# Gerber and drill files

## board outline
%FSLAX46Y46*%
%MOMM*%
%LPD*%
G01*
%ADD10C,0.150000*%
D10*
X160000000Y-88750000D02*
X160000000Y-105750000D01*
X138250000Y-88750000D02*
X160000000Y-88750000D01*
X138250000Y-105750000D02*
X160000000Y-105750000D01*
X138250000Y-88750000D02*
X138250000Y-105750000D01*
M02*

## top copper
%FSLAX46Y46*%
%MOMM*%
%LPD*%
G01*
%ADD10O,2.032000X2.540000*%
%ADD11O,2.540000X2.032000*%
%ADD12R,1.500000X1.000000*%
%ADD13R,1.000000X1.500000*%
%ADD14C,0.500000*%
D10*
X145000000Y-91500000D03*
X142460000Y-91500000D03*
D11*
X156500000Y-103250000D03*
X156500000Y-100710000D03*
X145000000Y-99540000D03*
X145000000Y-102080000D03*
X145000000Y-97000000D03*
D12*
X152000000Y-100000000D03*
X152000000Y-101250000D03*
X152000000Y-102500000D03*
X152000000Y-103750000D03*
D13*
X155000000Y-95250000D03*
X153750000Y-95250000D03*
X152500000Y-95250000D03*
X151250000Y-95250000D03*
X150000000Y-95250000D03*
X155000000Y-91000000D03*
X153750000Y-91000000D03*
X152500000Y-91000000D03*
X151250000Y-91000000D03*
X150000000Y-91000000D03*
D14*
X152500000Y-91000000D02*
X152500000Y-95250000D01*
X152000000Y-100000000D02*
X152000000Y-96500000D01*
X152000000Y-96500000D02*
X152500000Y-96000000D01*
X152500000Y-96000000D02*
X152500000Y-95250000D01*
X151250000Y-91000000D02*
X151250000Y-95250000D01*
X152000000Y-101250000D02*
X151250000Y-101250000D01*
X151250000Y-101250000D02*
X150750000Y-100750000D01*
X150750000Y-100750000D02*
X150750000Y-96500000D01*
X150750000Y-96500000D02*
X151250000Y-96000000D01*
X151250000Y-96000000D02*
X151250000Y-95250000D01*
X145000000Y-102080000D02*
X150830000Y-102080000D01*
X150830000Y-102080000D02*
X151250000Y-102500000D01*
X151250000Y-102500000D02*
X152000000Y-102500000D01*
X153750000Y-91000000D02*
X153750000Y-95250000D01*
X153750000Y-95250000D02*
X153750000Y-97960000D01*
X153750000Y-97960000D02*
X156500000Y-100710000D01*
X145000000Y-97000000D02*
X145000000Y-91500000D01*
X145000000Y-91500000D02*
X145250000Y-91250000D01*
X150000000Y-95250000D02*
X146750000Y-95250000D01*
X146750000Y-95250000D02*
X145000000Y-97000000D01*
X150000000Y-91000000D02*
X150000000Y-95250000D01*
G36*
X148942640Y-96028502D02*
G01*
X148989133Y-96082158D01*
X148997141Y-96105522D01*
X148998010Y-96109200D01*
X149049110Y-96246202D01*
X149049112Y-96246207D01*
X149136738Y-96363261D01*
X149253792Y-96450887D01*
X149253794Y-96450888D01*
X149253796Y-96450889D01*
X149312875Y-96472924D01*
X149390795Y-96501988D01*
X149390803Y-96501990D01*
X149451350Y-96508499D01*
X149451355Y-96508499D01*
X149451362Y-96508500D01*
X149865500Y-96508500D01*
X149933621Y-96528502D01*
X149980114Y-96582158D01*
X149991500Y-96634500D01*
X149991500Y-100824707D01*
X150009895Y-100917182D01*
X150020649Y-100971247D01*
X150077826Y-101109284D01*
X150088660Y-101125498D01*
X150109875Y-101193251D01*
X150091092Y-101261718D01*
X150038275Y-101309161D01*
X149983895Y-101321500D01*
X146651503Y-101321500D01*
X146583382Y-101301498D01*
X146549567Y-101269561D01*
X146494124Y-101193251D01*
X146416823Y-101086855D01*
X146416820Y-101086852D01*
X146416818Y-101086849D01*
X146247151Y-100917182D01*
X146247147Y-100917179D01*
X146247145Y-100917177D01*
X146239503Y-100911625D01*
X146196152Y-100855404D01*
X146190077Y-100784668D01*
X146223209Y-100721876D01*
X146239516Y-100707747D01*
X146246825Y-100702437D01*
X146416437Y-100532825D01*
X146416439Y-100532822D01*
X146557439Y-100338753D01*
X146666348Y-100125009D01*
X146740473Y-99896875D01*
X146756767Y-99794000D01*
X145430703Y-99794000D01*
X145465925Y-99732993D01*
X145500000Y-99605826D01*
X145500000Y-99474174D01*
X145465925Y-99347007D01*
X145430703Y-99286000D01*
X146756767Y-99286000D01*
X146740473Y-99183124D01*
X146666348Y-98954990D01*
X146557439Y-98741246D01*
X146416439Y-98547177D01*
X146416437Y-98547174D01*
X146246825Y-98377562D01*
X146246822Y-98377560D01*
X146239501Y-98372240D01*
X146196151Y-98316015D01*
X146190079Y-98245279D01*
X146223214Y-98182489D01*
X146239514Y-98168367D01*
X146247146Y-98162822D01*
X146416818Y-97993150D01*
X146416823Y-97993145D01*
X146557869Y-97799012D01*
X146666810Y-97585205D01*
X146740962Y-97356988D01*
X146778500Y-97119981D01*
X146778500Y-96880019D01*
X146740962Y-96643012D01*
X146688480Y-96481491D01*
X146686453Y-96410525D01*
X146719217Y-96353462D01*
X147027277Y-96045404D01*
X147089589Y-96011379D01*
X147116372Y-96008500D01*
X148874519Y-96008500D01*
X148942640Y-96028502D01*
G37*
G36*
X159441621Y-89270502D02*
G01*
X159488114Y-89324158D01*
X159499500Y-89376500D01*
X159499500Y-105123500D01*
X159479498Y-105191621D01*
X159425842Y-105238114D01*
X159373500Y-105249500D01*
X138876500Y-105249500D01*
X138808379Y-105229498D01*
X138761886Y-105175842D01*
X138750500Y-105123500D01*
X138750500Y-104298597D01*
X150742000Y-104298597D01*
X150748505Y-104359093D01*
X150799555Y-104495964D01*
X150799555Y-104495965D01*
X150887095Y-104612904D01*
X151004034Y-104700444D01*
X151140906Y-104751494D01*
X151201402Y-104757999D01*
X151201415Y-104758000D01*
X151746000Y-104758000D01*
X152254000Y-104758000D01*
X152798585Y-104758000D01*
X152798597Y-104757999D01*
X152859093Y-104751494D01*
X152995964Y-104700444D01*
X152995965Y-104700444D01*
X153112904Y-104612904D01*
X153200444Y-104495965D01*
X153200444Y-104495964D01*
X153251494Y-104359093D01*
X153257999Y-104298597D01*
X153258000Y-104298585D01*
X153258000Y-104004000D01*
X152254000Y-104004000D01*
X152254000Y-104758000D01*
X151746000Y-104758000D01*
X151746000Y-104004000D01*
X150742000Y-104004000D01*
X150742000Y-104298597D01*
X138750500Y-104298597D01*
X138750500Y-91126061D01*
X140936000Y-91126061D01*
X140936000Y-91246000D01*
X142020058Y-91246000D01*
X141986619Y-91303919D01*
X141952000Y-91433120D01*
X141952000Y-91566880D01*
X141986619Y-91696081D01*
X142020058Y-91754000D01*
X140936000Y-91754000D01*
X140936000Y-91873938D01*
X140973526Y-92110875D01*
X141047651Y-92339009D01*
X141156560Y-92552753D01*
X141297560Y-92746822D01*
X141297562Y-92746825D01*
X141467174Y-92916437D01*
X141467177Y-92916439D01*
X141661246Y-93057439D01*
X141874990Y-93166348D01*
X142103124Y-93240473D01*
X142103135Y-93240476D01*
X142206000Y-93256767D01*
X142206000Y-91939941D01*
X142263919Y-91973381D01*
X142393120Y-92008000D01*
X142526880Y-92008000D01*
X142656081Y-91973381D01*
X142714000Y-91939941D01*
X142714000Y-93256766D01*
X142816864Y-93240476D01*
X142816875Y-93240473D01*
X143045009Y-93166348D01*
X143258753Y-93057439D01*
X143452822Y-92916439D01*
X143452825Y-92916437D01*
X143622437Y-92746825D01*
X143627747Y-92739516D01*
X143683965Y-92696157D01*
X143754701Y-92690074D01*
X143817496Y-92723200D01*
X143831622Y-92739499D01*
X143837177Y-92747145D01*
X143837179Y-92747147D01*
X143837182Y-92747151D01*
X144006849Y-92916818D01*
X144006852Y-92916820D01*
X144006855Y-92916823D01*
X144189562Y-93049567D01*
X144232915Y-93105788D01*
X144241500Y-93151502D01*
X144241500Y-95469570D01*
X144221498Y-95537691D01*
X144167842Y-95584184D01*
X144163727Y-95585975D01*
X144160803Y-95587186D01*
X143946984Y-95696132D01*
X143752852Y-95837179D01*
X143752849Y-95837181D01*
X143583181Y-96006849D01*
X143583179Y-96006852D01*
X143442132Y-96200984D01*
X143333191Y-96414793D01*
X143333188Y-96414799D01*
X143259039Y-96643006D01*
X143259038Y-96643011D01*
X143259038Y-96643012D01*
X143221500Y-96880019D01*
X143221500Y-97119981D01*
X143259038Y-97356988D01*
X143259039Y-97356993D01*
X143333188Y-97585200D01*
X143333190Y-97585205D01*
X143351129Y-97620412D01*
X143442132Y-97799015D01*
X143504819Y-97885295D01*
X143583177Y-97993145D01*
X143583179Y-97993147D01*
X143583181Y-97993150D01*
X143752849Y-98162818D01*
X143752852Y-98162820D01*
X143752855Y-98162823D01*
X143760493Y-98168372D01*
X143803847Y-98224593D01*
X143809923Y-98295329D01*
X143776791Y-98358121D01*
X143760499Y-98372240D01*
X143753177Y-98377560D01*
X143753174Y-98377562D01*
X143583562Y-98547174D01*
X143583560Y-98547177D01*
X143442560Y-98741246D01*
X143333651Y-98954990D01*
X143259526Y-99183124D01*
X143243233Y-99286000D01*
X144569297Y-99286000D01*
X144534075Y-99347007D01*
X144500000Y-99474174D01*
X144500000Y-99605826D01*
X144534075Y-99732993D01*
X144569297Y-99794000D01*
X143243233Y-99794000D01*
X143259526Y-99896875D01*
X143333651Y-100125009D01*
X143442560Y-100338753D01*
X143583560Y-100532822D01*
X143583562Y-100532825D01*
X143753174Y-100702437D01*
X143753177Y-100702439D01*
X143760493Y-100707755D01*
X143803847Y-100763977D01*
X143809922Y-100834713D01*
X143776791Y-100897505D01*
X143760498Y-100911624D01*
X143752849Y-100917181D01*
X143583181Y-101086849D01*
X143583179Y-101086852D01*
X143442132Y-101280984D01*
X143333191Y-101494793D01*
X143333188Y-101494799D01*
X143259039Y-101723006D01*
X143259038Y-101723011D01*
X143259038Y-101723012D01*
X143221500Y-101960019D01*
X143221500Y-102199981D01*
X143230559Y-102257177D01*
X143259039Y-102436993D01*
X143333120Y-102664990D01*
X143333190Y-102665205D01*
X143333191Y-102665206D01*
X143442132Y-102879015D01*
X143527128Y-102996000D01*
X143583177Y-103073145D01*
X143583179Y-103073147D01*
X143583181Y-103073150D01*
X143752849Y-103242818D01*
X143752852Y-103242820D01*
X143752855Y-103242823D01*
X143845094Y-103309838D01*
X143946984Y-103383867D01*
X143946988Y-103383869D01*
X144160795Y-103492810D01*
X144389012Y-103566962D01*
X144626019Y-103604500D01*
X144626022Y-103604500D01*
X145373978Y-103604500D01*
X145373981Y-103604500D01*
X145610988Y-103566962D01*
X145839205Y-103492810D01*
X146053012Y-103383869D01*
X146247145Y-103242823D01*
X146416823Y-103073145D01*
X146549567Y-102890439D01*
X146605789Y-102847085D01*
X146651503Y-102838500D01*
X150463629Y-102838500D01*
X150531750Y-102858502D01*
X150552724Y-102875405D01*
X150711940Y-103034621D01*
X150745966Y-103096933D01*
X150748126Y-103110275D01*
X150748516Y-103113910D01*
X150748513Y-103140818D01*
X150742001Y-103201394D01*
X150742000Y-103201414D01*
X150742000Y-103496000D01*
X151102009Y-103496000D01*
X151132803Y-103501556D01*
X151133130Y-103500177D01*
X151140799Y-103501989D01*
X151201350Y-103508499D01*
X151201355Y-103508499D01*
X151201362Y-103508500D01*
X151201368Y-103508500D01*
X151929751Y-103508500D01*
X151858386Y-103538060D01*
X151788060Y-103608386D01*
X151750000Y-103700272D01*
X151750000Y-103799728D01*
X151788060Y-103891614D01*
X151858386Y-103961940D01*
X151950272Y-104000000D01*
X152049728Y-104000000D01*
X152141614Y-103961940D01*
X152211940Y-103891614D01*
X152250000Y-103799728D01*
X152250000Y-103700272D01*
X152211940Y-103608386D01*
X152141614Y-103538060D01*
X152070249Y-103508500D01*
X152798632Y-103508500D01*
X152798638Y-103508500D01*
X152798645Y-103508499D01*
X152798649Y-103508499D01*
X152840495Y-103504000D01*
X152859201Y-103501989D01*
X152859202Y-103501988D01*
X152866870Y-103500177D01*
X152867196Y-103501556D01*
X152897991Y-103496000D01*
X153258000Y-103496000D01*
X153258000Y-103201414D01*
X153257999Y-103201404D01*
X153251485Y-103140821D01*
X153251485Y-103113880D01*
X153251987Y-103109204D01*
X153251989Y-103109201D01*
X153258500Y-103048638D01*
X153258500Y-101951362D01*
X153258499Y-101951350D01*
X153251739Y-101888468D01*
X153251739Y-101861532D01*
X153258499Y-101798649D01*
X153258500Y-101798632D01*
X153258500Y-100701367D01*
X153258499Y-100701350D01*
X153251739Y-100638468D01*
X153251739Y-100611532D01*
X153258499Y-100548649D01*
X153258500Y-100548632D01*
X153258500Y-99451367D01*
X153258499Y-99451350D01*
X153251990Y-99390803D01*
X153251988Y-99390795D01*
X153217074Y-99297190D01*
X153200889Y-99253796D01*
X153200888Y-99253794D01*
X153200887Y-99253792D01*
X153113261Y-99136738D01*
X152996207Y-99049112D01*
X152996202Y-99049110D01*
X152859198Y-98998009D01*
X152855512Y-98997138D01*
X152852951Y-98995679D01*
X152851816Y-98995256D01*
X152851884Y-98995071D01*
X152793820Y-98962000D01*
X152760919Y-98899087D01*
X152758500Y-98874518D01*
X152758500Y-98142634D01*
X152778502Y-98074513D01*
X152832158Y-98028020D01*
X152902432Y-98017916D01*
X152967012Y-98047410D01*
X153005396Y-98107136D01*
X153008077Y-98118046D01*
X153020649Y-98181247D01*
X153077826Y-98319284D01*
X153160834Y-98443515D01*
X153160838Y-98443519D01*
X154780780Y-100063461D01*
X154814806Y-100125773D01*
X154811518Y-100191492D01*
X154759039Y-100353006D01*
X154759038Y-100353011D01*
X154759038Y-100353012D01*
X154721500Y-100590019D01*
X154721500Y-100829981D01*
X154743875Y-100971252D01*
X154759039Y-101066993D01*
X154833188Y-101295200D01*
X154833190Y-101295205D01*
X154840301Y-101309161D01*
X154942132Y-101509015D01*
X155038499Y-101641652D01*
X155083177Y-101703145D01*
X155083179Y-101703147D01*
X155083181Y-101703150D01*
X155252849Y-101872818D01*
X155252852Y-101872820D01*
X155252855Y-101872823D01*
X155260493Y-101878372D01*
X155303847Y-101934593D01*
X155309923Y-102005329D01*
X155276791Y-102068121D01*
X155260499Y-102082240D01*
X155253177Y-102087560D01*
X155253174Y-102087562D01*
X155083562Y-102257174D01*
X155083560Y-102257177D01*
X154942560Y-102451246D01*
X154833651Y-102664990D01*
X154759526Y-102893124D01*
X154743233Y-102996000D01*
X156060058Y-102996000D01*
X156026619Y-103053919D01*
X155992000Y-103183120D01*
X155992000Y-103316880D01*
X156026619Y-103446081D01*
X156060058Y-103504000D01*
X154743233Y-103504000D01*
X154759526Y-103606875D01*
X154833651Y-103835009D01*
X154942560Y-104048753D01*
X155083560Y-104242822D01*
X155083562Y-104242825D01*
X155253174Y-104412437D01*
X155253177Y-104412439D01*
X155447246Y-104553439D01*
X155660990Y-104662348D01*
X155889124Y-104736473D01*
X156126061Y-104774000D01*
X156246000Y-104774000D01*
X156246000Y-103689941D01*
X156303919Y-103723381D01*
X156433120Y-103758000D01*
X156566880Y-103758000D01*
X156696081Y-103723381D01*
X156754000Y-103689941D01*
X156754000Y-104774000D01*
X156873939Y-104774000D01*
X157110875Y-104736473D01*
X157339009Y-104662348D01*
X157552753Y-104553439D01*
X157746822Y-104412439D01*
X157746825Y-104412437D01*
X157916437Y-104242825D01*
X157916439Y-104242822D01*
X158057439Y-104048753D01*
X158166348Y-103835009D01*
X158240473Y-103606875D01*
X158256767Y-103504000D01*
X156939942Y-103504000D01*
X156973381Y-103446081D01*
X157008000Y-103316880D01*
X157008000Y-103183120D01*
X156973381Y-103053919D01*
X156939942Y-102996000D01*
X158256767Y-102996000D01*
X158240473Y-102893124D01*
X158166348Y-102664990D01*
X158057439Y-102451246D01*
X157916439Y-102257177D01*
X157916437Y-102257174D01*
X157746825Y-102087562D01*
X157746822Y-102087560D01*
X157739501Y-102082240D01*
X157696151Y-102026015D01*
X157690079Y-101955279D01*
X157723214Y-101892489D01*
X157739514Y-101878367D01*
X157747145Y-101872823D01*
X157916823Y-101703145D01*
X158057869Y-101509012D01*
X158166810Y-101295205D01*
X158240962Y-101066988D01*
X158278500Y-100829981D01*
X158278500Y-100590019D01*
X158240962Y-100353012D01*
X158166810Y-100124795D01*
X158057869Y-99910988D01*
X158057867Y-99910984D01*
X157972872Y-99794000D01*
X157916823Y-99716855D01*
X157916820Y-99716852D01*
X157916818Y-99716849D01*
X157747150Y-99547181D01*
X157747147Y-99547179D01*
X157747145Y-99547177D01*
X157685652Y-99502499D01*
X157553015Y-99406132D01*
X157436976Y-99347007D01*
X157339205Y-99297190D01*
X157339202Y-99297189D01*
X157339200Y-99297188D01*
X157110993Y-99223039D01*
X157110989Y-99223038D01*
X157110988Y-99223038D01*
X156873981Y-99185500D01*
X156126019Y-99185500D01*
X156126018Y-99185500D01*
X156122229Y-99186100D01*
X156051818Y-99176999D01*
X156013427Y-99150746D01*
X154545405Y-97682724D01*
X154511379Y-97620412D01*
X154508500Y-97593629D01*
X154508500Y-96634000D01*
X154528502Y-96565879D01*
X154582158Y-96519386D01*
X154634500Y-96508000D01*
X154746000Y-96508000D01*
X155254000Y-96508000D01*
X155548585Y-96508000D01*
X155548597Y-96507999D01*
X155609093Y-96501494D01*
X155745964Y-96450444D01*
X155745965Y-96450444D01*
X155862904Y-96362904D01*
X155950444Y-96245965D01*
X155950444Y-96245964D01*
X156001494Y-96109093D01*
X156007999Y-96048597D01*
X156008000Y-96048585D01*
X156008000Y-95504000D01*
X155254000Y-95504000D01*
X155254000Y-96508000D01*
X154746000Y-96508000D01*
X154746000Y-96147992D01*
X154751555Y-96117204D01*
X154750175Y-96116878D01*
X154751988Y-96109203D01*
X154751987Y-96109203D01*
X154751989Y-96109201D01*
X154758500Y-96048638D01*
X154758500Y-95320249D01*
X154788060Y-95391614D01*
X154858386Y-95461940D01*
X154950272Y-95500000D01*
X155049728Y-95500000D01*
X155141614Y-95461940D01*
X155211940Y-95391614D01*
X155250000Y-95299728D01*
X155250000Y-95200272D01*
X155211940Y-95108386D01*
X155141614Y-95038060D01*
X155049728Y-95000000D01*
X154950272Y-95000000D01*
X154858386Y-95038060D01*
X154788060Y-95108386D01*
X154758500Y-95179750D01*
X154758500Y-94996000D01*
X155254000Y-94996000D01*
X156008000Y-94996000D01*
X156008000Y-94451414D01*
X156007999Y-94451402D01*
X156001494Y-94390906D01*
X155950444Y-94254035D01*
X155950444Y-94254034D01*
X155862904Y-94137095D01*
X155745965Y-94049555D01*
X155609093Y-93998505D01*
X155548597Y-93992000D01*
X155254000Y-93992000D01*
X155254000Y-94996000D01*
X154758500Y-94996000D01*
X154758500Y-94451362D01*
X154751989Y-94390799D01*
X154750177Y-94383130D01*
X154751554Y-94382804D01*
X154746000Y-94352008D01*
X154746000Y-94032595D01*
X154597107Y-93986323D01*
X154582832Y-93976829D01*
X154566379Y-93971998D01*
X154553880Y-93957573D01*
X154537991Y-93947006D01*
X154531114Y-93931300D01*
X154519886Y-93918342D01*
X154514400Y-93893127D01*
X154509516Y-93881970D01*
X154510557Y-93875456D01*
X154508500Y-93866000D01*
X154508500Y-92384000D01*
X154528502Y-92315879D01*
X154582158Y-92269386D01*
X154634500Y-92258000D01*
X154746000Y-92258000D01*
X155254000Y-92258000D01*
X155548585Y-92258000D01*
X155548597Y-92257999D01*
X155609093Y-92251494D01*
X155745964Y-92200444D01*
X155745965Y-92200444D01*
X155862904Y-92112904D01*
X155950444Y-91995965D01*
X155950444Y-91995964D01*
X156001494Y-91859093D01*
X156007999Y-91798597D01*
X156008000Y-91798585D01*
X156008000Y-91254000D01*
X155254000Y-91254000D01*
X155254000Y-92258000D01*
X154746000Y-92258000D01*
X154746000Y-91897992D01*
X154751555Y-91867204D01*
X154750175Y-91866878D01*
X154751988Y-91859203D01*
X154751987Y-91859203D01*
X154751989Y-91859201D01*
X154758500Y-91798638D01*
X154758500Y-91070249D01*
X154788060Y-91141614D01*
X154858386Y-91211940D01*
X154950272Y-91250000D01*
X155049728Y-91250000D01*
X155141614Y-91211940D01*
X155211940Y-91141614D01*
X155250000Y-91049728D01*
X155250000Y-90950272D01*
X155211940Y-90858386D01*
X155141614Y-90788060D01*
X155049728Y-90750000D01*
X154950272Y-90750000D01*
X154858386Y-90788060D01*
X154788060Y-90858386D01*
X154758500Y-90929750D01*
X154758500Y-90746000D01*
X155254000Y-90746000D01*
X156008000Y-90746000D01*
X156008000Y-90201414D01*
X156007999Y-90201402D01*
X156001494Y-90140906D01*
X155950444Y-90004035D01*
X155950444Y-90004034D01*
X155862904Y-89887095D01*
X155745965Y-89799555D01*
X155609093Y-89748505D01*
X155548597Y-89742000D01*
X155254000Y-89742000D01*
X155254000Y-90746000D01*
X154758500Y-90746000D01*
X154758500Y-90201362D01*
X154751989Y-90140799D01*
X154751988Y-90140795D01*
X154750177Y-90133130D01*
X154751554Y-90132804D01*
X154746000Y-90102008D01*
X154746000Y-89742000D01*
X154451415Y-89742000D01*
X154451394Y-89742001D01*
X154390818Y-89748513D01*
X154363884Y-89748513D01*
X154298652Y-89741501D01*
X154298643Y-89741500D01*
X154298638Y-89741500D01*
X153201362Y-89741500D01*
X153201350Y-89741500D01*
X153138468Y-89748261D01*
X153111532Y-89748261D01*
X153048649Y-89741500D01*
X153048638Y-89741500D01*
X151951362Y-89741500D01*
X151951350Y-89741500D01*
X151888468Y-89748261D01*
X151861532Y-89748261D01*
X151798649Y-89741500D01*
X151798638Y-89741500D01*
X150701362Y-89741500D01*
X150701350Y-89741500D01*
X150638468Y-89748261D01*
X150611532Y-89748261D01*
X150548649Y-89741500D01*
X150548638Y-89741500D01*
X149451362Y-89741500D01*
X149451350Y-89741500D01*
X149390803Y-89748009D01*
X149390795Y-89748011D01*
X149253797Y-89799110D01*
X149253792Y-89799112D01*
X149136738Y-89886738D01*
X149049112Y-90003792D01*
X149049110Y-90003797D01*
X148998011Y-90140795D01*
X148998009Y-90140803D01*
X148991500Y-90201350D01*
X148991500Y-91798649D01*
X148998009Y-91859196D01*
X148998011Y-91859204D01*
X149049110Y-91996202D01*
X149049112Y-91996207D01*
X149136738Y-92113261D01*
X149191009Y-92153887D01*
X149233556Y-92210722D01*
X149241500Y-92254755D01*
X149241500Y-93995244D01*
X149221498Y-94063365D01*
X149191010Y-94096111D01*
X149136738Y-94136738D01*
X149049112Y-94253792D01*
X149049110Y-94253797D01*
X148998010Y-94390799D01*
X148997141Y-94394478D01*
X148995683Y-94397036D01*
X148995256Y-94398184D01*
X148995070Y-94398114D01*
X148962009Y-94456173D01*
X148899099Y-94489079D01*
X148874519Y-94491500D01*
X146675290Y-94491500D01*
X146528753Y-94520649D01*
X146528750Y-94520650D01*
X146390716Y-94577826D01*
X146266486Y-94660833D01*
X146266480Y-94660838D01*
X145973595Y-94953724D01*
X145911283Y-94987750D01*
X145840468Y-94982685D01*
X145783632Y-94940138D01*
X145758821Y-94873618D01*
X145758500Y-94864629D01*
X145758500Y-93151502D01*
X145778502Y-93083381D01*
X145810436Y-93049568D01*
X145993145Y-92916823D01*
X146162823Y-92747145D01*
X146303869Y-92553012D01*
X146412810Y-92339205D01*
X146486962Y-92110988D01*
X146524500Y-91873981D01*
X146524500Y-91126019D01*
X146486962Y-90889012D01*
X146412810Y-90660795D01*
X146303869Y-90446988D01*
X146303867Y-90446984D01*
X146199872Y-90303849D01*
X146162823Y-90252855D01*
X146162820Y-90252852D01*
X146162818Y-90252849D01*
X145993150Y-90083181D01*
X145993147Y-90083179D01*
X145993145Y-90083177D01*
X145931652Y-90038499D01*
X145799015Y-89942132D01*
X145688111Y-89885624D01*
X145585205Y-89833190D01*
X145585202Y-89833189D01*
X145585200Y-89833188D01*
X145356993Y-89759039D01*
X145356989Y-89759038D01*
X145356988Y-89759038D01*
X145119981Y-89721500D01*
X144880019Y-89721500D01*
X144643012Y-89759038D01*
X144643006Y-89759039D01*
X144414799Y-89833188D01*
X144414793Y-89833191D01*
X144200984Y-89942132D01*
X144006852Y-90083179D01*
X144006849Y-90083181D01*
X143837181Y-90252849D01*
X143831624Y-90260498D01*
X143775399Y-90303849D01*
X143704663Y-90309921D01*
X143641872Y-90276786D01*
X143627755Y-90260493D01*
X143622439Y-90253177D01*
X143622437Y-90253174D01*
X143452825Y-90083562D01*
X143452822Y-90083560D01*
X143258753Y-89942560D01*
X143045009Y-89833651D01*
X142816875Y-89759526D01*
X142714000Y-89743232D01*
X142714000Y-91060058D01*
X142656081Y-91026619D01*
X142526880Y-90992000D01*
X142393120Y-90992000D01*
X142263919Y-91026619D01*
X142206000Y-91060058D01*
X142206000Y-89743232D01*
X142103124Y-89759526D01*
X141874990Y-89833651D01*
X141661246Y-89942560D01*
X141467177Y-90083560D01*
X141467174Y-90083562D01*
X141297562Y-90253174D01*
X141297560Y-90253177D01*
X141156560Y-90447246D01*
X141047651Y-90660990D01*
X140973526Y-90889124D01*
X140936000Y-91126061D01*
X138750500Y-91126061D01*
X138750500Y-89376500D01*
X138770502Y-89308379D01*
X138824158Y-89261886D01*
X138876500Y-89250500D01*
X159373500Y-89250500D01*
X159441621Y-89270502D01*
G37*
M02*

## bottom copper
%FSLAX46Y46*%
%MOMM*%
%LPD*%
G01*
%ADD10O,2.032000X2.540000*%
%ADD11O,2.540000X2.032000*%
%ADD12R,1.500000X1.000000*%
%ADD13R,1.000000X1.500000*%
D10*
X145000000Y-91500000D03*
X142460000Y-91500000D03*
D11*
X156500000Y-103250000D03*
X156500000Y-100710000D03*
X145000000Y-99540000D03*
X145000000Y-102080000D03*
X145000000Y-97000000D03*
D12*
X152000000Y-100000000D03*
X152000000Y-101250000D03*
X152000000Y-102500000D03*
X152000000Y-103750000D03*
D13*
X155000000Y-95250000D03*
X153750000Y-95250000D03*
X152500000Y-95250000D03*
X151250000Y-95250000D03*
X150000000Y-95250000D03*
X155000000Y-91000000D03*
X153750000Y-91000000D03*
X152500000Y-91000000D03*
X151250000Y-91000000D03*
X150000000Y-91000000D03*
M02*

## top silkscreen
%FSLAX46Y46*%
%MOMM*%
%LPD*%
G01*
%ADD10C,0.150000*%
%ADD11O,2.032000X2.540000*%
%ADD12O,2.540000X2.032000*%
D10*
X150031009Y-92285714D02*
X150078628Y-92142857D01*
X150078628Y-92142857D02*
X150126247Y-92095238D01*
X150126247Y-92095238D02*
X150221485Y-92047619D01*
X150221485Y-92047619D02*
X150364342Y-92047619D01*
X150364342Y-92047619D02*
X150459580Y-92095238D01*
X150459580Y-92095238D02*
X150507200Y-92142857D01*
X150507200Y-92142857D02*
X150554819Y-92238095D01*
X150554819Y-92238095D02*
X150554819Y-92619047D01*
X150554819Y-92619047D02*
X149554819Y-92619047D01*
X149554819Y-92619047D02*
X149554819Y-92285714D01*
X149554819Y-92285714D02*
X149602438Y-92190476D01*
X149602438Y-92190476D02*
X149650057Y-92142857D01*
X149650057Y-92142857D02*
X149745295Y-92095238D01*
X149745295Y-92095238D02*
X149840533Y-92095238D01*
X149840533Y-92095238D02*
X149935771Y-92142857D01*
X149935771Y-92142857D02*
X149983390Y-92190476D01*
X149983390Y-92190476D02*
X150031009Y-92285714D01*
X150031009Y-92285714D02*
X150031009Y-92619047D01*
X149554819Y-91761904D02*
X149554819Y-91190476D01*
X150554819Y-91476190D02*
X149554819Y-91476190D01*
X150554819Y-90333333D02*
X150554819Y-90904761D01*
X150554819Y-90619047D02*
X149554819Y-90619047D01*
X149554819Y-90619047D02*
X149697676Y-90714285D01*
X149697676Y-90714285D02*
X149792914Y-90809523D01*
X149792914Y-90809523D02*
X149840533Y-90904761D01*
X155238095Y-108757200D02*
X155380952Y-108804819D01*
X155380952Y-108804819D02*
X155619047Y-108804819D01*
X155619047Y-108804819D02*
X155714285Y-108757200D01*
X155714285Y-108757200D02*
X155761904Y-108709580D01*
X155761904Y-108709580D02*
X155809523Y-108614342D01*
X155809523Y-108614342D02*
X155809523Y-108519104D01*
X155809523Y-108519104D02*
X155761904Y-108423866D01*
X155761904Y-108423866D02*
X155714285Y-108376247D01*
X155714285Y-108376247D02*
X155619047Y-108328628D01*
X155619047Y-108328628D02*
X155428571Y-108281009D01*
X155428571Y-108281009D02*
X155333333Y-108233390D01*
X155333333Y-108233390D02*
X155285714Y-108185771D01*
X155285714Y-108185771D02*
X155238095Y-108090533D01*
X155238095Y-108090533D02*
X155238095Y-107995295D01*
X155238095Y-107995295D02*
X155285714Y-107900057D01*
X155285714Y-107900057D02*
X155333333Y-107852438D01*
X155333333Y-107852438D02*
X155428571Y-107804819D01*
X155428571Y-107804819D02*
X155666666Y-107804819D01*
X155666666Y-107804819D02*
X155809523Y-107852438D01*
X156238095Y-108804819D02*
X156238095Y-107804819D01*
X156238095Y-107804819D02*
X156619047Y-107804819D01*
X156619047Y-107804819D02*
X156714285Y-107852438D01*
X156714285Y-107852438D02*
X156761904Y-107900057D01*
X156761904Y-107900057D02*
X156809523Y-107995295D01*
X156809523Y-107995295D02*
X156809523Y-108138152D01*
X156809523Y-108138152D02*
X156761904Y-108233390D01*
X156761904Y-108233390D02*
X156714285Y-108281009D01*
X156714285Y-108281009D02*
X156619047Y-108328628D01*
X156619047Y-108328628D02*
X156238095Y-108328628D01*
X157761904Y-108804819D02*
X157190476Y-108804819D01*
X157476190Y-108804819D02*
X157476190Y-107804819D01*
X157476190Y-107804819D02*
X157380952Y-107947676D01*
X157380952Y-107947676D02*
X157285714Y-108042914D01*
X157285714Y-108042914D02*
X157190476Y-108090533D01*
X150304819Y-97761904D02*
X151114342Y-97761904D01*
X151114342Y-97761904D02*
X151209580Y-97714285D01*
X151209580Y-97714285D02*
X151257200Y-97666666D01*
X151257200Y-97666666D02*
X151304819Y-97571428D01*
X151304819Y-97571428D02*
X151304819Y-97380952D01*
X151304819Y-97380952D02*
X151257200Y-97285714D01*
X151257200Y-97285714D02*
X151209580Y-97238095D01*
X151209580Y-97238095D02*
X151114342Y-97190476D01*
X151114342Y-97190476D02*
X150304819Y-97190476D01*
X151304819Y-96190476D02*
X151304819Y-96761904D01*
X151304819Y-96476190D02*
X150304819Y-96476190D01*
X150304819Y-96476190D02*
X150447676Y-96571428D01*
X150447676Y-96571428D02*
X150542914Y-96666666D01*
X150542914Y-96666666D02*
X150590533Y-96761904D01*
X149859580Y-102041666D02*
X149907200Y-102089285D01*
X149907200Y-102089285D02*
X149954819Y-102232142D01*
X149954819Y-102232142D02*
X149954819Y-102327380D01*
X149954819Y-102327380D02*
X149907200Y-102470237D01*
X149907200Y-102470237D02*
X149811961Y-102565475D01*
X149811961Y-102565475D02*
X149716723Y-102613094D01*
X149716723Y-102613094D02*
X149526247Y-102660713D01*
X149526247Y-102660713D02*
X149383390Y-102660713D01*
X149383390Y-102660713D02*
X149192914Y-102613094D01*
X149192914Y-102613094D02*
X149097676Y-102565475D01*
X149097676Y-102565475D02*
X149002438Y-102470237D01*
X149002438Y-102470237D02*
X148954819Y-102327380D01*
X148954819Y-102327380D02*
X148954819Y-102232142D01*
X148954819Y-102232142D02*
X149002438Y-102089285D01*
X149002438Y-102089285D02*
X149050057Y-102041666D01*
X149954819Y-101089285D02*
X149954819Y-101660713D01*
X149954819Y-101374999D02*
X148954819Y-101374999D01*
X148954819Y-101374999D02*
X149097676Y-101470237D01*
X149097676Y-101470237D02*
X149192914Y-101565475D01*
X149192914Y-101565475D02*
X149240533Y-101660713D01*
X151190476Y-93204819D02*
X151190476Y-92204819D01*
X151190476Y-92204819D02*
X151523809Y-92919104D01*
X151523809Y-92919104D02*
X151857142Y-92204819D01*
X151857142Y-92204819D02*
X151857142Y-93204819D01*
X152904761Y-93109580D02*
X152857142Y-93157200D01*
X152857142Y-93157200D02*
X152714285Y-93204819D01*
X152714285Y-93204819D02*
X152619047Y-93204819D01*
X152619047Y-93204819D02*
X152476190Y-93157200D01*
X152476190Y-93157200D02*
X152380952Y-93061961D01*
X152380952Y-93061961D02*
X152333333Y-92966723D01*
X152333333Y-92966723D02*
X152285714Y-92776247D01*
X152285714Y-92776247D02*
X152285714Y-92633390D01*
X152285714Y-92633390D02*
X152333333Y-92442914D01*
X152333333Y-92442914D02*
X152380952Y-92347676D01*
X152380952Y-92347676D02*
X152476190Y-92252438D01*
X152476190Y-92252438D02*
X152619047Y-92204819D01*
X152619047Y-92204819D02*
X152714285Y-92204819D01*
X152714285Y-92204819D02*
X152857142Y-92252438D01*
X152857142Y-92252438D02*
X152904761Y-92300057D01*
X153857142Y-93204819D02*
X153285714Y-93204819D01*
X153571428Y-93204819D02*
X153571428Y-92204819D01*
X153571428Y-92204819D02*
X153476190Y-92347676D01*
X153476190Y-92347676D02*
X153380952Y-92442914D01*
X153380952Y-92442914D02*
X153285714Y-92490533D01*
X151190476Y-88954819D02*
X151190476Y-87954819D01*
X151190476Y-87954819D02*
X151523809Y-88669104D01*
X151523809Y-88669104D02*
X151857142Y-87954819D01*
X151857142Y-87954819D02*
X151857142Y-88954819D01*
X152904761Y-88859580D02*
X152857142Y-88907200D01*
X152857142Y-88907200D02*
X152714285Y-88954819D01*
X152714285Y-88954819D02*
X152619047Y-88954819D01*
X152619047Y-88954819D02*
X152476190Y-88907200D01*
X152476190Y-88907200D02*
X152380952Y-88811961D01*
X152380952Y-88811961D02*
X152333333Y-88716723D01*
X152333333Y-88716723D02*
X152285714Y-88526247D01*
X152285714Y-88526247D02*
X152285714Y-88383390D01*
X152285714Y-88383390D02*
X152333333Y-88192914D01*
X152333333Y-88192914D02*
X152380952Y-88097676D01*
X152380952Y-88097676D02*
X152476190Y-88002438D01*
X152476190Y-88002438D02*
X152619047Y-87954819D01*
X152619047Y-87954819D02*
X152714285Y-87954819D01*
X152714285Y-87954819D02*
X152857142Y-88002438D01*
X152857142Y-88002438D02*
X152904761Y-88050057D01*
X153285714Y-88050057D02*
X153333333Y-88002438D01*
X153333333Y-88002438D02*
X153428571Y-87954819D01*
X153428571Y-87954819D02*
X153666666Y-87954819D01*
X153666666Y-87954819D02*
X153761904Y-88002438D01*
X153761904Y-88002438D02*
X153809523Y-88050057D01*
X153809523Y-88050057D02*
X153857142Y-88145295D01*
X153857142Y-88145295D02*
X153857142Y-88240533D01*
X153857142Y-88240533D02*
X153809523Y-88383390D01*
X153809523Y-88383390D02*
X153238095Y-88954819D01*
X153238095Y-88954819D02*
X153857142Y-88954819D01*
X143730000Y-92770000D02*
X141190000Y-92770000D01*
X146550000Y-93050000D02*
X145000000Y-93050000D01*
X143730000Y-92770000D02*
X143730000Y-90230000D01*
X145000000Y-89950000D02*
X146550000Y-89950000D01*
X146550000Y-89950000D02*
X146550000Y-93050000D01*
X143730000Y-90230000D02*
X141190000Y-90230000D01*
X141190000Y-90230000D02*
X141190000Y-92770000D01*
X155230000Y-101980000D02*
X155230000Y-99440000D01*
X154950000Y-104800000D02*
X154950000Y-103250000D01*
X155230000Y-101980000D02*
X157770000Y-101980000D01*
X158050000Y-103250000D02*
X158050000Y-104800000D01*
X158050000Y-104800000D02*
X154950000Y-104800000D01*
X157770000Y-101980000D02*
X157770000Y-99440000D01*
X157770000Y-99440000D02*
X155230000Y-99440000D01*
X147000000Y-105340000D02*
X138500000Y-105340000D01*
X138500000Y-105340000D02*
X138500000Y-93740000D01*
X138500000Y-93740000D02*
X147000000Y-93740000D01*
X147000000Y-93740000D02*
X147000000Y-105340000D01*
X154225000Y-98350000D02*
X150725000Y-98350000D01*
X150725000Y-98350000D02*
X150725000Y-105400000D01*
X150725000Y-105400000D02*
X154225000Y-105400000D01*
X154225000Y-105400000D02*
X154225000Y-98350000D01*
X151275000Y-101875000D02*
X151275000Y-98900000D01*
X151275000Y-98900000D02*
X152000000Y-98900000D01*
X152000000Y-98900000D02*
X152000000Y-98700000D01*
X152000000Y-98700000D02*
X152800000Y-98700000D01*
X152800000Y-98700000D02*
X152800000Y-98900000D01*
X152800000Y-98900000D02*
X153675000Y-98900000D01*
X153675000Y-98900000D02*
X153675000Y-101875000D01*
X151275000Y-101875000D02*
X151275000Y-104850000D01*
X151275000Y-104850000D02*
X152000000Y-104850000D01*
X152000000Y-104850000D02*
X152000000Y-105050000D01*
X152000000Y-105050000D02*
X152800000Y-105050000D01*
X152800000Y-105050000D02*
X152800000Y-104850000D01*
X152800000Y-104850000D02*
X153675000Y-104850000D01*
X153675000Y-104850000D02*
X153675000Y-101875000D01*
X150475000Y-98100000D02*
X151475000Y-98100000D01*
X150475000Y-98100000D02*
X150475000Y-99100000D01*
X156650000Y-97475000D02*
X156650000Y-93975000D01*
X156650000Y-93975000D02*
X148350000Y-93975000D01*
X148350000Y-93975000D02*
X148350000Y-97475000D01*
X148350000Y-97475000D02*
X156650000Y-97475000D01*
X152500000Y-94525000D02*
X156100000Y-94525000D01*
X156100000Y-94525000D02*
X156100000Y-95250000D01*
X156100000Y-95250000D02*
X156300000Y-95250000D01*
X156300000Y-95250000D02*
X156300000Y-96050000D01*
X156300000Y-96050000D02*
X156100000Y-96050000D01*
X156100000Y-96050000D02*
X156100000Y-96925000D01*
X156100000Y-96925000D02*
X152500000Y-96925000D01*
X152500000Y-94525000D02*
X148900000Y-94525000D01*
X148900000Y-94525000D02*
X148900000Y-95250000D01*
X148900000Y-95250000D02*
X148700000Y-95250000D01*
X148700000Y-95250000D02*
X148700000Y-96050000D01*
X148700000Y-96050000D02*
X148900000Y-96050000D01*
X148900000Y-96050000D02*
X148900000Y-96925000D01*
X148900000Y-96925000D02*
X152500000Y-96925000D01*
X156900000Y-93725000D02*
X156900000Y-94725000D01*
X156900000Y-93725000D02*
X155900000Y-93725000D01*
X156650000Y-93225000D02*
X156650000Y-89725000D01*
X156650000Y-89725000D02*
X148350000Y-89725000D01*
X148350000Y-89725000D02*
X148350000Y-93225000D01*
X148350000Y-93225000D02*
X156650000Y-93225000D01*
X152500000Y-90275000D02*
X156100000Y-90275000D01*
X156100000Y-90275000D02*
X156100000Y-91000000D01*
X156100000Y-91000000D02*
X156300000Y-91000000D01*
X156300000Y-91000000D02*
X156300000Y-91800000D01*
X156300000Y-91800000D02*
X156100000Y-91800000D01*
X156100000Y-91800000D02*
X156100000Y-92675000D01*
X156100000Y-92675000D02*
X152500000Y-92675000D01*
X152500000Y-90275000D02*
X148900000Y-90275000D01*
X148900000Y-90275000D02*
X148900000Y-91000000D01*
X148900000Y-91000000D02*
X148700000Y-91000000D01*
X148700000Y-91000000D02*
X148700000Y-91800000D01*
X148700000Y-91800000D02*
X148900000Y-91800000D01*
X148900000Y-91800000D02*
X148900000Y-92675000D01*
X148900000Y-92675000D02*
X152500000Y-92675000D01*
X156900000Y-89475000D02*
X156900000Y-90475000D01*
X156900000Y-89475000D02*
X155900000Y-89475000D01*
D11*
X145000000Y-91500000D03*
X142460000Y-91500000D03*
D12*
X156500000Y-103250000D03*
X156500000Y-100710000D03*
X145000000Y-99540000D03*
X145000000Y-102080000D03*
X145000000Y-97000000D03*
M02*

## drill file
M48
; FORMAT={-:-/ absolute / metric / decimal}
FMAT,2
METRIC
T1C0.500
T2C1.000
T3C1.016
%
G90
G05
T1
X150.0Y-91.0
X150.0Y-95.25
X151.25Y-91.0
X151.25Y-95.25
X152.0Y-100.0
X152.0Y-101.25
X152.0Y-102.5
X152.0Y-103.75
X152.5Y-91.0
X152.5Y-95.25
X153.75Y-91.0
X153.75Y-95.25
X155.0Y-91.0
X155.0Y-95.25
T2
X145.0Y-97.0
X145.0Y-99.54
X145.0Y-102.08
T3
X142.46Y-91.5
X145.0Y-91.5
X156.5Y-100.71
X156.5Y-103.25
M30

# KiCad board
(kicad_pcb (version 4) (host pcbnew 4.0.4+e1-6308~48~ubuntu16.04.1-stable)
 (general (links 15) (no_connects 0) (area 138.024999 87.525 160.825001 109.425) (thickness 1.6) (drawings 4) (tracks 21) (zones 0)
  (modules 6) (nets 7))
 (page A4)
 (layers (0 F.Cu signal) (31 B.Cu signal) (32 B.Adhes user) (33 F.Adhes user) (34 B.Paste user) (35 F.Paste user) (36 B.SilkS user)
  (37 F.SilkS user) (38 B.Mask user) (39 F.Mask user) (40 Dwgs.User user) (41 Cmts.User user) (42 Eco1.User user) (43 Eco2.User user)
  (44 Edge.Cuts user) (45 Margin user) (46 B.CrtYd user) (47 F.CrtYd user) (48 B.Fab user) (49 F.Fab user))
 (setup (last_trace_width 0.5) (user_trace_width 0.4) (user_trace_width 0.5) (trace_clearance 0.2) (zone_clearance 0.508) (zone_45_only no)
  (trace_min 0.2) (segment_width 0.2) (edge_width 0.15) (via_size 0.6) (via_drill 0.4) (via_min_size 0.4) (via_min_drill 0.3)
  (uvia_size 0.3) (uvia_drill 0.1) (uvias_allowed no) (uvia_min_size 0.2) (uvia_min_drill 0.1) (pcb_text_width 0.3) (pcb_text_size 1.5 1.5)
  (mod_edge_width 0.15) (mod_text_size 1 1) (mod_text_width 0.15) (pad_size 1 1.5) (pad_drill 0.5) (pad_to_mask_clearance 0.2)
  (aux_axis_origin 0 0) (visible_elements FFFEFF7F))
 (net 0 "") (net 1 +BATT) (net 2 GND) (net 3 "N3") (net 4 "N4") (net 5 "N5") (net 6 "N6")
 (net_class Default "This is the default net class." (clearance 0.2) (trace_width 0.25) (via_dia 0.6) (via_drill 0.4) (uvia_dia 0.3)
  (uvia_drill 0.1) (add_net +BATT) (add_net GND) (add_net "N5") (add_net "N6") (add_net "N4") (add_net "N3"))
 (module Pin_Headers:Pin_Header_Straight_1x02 (layer F.Cu) (at 145 91.5 270)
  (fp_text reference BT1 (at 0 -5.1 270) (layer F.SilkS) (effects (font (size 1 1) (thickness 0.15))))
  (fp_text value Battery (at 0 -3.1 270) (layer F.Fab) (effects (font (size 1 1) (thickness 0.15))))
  (fp_line (start 1.27 1.27) (end 1.27 3.81) (layer F.SilkS) (width 0.15))
  (fp_line (start 1.55 -1.55) (end 1.55 0) (layer F.SilkS) (width 0.15))
  (fp_line (start 1.27 1.27) (end -1.27 1.27) (layer F.SilkS) (width 0.15))
  (fp_line (start -1.55 0) (end -1.55 -1.55) (layer F.SilkS) (width 0.15))
  (fp_line (start -1.55 -1.55) (end 1.55 -1.55) (layer F.SilkS) (width 0.15))
  (fp_line (start -1.27 1.27) (end -1.27 3.81) (layer F.SilkS) (width 0.15))
  (fp_line (start -1.27 3.81) (end 1.27 3.81) (layer F.SilkS) (width 0.15))
  (pad 1 thru_hole oval (at 0 0 270) (size 2.54 2.032) (drill 1.016) (layers *.Cu *.Mask F.SilkS) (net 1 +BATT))
  (pad 2 thru_hole oval (at 0 2.54 270) (size 2.54 2.032) (drill 1.016) (layers *.Cu *.Mask F.SilkS) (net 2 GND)))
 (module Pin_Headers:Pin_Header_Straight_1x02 (layer F.Cu) (at 156.5 103.25 180)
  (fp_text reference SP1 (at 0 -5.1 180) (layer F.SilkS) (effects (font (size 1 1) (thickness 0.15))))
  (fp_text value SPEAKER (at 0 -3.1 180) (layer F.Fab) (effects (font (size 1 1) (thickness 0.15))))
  (fp_line (start 1.27 1.27) (end 1.27 3.81) (layer F.SilkS) (width 0.15))
  (fp_line (start 1.55 -1.55) (end 1.55 0) (layer F.SilkS) (width 0.15))
  (fp_line (start 1.27 1.27) (end -1.27 1.27) (layer F.SilkS) (width 0.15))
  (fp_line (start -1.55 0) (end -1.55 -1.55) (layer F.SilkS) (width 0.15))
  (fp_line (start -1.55 -1.55) (end 1.55 -1.55) (layer F.SilkS) (width 0.15))
  (fp_line (start -1.27 1.27) (end -1.27 3.81) (layer F.SilkS) (width 0.15))
  (fp_line (start -1.27 3.81) (end 1.27 3.81) (layer F.SilkS) (width 0.15))
  (pad 1 thru_hole oval (at 0 0 180) (size 2.54 2.032) (drill 1.016) (layers *.Cu *.Mask F.SilkS) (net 2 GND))
  (pad 2 thru_hole oval (at 0 2.54 180) (size 2.54 2.032) (drill 1.016) (layers *.Cu *.Mask F.SilkS) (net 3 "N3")))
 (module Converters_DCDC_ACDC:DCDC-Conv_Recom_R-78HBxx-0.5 (layer F.Cu) (at 145 97 270)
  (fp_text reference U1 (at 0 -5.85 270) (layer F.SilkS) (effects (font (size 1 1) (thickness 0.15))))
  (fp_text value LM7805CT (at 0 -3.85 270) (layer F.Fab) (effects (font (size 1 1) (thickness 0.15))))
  (fp_line (start 8.34 -2) (end 8.34 6.5) (layer F.SilkS) (width 0.15))
  (fp_line (start 8.34 6.5) (end -3.26 6.5) (layer F.SilkS) (width 0.15))
  (fp_line (start -3.26 6.5) (end -3.26 -2) (layer F.SilkS) (width 0.15))
  (fp_line (start -3.26 -2) (end 8.34 -2) (layer F.SilkS) (width 0.15))
  (pad 2 thru_hole oval (at 2.54 0 270) (size 2.032 2.54) (drill 1) (layers *.Cu *.Mask F.SilkS) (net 2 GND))
  (pad 3 thru_hole oval (at 5.08 0 270) (size 2.032 2.54) (drill 1) (layers *.Cu *.Mask F.SilkS) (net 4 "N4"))
  (pad 1 thru_hole oval (at 0 0 270) (size 2.032 2.54) (drill 1) (layers *.Cu *.Mask F.SilkS) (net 1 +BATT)))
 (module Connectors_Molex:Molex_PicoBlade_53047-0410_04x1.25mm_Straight (layer F.Cu) (at 152 100 270)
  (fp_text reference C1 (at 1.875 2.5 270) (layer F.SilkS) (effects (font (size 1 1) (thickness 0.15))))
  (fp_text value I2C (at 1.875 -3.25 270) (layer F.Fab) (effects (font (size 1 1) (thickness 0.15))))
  (fp_line (start -1.65 -2.225) (end -1.65 1.275) (layer F.SilkS) (width 0.15))
  (fp_line (start -1.65 1.275) (end 5.4 1.275) (layer F.SilkS) (width 0.15))
  (fp_line (start 5.4 1.275) (end 5.4 -2.225) (layer F.SilkS) (width 0.15))
  (fp_line (start 5.4 -2.225) (end -1.65 -2.225) (layer F.SilkS) (width 0.15))
  (fp_line (start 1.875 0.725) (end -1.1 0.725) (layer F.SilkS) (width 0.15))
  (fp_line (start -1.1 0.725) (end -1.1 0) (layer F.SilkS) (width 0.15))
  (fp_line (start -1.1 0) (end -1.3 0) (layer F.SilkS) (width 0.15))
  (fp_line (start -1.3 0) (end -1.3 -0.8) (layer F.SilkS) (width 0.15))
  (fp_line (start -1.3 -0.8) (end -1.1 -0.8) (layer F.SilkS) (width 0.15))
  (fp_line (start -1.1 -0.8) (end -1.1 -1.675) (layer F.SilkS) (width 0.15))
  (fp_line (start -1.1 -1.675) (end 1.875 -1.675) (layer F.SilkS) (width 0.15))
  (fp_line (start 1.875 0.725) (end 4.85 0.725) (layer F.SilkS) (width 0.15))
  (fp_line (start 4.85 0.725) (end 4.85 0) (layer F.SilkS) (width 0.15))
  (fp_line (start 4.85 0) (end 5.05 0) (layer F.SilkS) (width 0.15))
  (fp_line (start 5.05 0) (end 5.05 -0.8) (layer F.SilkS) (width 0.15))
  (fp_line (start 5.05 -0.8) (end 4.85 -0.8) (layer F.SilkS) (width 0.15))
  (fp_line (start 4.85 -0.8) (end 4.85 -1.675) (layer F.SilkS) (width 0.15))
  (fp_line (start 4.85 -1.675) (end 1.875 -1.675) (layer F.SilkS) (width 0.15))
  (fp_line (start -1.9 1.525) (end -1.9 0.525) (layer F.SilkS) (width 0.15))
  (fp_line (start -1.9 1.525) (end -0.9 1.525) (layer F.SilkS) (width 0.15))
  (pad 1 thru_hole rect (at 0 0 270) (size 1 1.5) (drill 0.5) (layers *.Cu *.Mask) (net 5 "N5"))
  (pad 2 thru_hole rect (at 1.25 0 270) (size 1 1.5) (drill 0.5) (layers *.Cu *.Mask) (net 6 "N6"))
  (pad 3 thru_hole rect (at 2.5 0 270) (size 1 1.5) (drill 0.5) (layers *.Cu *.Mask) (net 4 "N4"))
  (pad 4 thru_hole rect (at 3.75 0 270) (size 1 1.5) (drill 0.5) (layers *.Cu *.Mask) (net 2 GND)))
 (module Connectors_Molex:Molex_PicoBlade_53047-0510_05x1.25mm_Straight (layer F.Cu) (at 155 95.25 180)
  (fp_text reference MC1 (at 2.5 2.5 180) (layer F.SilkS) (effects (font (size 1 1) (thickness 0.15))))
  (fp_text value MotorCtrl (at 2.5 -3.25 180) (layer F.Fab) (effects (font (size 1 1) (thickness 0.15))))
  (fp_line (start -1.65 -2.225) (end -1.65 1.275) (layer F.SilkS) (width 0.15))
  (fp_line (start -1.65 1.275) (end 6.65 1.275) (layer F.SilkS) (width 0.15))
  (fp_line (start 6.65 1.275) (end 6.65 -2.225) (layer F.SilkS) (width 0.15))
  (fp_line (start 6.65 -2.225) (end -1.65 -2.225) (layer F.SilkS) (width 0.15))
  (fp_line (start 2.5 0.725) (end -1.1 0.725) (layer F.SilkS) (width 0.15))
  (fp_line (start -1.1 0.725) (end -1.1 0) (layer F.SilkS) (width 0.15))
  (fp_line (start -1.1 0) (end -1.3 0) (layer F.SilkS) (width 0.15))
  (fp_line (start -1.3 0) (end -1.3 -0.8) (layer F.SilkS) (width 0.15))
  (fp_line (start -1.3 -0.8) (end -1.1 -0.8) (layer F.SilkS) (width 0.15))
  (fp_line (start -1.1 -0.8) (end -1.1 -1.675) (layer F.SilkS) (width 0.15))
  (fp_line (start -1.1 -1.675) (end 2.5 -1.675) (layer F.SilkS) (width 0.15))
  (fp_line (start 2.5 0.725) (end 6.1 0.725) (layer F.SilkS) (width 0.15))
  (fp_line (start 6.1 0.725) (end 6.1 0) (layer F.SilkS) (width 0.15))
  (fp_line (start 6.1 0) (end 6.3 0) (layer F.SilkS) (width 0.15))
  (fp_line (start 6.3 0) (end 6.3 -0.8) (layer F.SilkS) (width 0.15))
  (fp_line (start 6.3 -0.8) (end 6.1 -0.8) (layer F.SilkS) (width 0.15))
  (fp_line (start 6.1 -0.8) (end 6.1 -1.675) (layer F.SilkS) (width 0.15))
  (fp_line (start 6.1 -1.675) (end 2.5 -1.675) (layer F.SilkS) (width 0.15))
  (fp_line (start -1.9 1.525) (end -1.9 0.525) (layer F.SilkS) (width 0.15))
  (fp_line (start -1.9 1.525) (end -0.9 1.525) (layer F.SilkS) (width 0.15))
  (pad 1 thru_hole rect (at 0 0 180) (size 1 1.5) (drill 0.5) (layers *.Cu *.Mask) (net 2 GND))
  (pad 2 thru_hole rect (at 1.25 0 180) (size 1 1.5) (drill 0.5) (layers *.Cu *.Mask) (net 3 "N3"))
  (pad 3 thru_hole rect (at 2.5 0 180) (size 1 1.5) (drill 0.5) (layers *.Cu *.Mask) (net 5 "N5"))
  (pad 4 thru_hole rect (at 3.75 0 180) (size 1 1.5) (drill 0.5) (layers *.Cu *.Mask) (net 6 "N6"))
  (pad 5 thru_hole rect (at 5 0 180) (size 1 1.5) (drill 0.5) (layers *.Cu *.Mask) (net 1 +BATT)))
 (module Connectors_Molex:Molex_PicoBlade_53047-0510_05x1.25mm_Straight (layer F.Cu) (at 155 91 180)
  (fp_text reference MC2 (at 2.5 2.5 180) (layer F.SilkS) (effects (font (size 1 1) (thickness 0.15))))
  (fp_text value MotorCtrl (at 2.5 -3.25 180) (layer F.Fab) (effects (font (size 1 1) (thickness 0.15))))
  (fp_line (start -1.65 -2.225) (end -1.65 1.275) (layer F.SilkS) (width 0.15))
  (fp_line (start -1.65 1.275) (end 6.65 1.275) (layer F.SilkS) (width 0.15))
  (fp_line (start 6.65 1.275) (end 6.65 -2.225) (layer F.SilkS) (width 0.15))
  (fp_line (start 6.65 -2.225) (end -1.65 -2.225) (layer F.SilkS) (width 0.15))
  (fp_line (start 2.5 0.725) (end -1.1 0.725) (layer F.SilkS) (width 0.15))
  (fp_line (start -1.1 0.725) (end -1.1 0) (layer F.SilkS) (width 0.15))
  (fp_line (start -1.1 0) (end -1.3 0) (layer F.SilkS) (width 0.15))
  (fp_line (start -1.3 0) (end -1.3 -0.8) (layer F.SilkS) (width 0.15))
  (fp_line (start -1.3 -0.8) (end -1.1 -0.8) (layer F.SilkS) (width 0.15))
  (fp_line (start -1.1 -0.8) (end -1.1 -1.675) (layer F.SilkS) (width 0.15))
  (fp_line (start -1.1 -1.675) (end 2.5 -1.675) (layer F.SilkS) (width 0.15))
  (fp_line (start 2.5 0.725) (end 6.1 0.725) (layer F.SilkS) (width 0.15))
  (fp_line (start 6.1 0.725) (end 6.1 0) (layer F.SilkS) (width 0.15))
  (fp_line (start 6.1 0) (end 6.3 0) (layer F.SilkS) (width 0.15))
  (fp_line (start 6.3 0) (end 6.3 -0.8) (layer F.SilkS) (width 0.15))
  (fp_line (start 6.3 -0.8) (end 6.1 -0.8) (layer F.SilkS) (width 0.15))
  (fp_line (start 6.1 -0.8) (end 6.1 -1.675) (layer F.SilkS) (width 0.15))
  (fp_line (start 6.1 -1.675) (end 2.5 -1.675) (layer F.SilkS) (width 0.15))
  (fp_line (start -1.9 1.525) (end -1.9 0.525) (layer F.SilkS) (width 0.15))
  (fp_line (start -1.9 1.525) (end -0.9 1.525) (layer F.SilkS) (width 0.15))
  (pad 1 thru_hole rect (at 0 0 180) (size 1 1.5) (drill 0.5) (layers *.Cu *.Mask) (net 2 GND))
  (pad 2 thru_hole rect (at 1.25 0 180) (size 1 1.5) (drill 0.5) (layers *.Cu *.Mask) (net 3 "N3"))
  (pad 3 thru_hole rect (at 2.5 0 180) (size 1 1.5) (drill 0.5) (layers *.Cu *.Mask) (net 5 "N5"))
  (pad 4 thru_hole rect (at 3.75 0 180) (size 1 1.5) (drill 0.5) (layers *.Cu *.Mask) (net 6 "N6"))
  (pad 5 thru_hole rect (at 5 0 180) (size 1 1.5) (drill 0.5) (layers *.Cu *.Mask) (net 1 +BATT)))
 (gr_line (start 160 88.75) (end 160 105.75) (angle 90) (layer Edge.Cuts) (width 0.15))
 (gr_line (start 138.25 88.75) (end 160 88.75) (angle 90) (layer Edge.Cuts) (width 0.15))
 (gr_line (start 138.25 105.75) (end 160 105.75) (angle 90) (layer Edge.Cuts) (width 0.15))
 (gr_line (start 138.25 88.75) (end 138.25 105.75) (angle 90) (layer Edge.Cuts) (width 0.15))
 (segment (start 152.5 91) (end 152.5 95.25) (width 0.5) (layer F.Cu) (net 5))
 (segment (start 152 100) (end 152 96.5) (width 0.5) (layer F.Cu) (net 5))
 (segment (start 152 96.5) (end 152.5 96) (width 0.5) (layer F.Cu) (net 5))
 (segment (start 152.5 96) (end 152.5 95.25) (width 0.5) (layer F.Cu) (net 5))
 (segment (start 151.25 91) (end 151.25 95.25) (width 0.5) (layer F.Cu) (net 6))
 (segment (start 152 101.25) (end 151.25 101.25) (width 0.5) (layer F.Cu) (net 6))
 (segment (start 151.25 101.25) (end 150.75 100.75) (width 0.5) (layer F.Cu) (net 6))
 (segment (start 150.75 100.75) (end 150.75 96.5) (width 0.5) (layer F.Cu) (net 6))
 (segment (start 150.75 96.5) (end 151.25 96) (width 0.5) (layer F.Cu) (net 6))
 (segment (start 151.25 96) (end 151.25 95.25) (width 0.5) (layer F.Cu) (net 6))
 (segment (start 145 102.08) (end 150.83 102.08) (width 0.5) (layer F.Cu) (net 4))
 (segment (start 150.83 102.08) (end 151.25 102.5) (width 0.5) (layer F.Cu) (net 4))
 (segment (start 151.25 102.5) (end 152 102.5) (width 0.5) (layer F.Cu) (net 4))
 (segment (start 153.75 91) (end 153.75 95.25) (width 0.5) (layer F.Cu) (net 3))
 (segment (start 153.75 95.25) (end 153.75 97.96) (width 0.5) (layer F.Cu) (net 3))
 (segment (start 153.75 97.96) (end 156.5 100.71) (width 0.5) (layer F.Cu) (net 3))
 (segment (start 145 97) (end 145 91.5) (width 0.5) (layer F.Cu) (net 1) (status C00000))
 (segment (start 145 91.5) (end 145.25 91.25) (width 0.5) (layer F.Cu) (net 1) (status C00000))
 (segment (start 150 95.25) (end 146.75 95.25) (width 0.5) (layer F.Cu) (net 1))
 (segment (start 146.75 95.25) (end 145 97) (width 0.5) (layer F.Cu) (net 1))
 (segment (start 150 91) (end 150 95.25) (width 0.5) (layer F.Cu) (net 1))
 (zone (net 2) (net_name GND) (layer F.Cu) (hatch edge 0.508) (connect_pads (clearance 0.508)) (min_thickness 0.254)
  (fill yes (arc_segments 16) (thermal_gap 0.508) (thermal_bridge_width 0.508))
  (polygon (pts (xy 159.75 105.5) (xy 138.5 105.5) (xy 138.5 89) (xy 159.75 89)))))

